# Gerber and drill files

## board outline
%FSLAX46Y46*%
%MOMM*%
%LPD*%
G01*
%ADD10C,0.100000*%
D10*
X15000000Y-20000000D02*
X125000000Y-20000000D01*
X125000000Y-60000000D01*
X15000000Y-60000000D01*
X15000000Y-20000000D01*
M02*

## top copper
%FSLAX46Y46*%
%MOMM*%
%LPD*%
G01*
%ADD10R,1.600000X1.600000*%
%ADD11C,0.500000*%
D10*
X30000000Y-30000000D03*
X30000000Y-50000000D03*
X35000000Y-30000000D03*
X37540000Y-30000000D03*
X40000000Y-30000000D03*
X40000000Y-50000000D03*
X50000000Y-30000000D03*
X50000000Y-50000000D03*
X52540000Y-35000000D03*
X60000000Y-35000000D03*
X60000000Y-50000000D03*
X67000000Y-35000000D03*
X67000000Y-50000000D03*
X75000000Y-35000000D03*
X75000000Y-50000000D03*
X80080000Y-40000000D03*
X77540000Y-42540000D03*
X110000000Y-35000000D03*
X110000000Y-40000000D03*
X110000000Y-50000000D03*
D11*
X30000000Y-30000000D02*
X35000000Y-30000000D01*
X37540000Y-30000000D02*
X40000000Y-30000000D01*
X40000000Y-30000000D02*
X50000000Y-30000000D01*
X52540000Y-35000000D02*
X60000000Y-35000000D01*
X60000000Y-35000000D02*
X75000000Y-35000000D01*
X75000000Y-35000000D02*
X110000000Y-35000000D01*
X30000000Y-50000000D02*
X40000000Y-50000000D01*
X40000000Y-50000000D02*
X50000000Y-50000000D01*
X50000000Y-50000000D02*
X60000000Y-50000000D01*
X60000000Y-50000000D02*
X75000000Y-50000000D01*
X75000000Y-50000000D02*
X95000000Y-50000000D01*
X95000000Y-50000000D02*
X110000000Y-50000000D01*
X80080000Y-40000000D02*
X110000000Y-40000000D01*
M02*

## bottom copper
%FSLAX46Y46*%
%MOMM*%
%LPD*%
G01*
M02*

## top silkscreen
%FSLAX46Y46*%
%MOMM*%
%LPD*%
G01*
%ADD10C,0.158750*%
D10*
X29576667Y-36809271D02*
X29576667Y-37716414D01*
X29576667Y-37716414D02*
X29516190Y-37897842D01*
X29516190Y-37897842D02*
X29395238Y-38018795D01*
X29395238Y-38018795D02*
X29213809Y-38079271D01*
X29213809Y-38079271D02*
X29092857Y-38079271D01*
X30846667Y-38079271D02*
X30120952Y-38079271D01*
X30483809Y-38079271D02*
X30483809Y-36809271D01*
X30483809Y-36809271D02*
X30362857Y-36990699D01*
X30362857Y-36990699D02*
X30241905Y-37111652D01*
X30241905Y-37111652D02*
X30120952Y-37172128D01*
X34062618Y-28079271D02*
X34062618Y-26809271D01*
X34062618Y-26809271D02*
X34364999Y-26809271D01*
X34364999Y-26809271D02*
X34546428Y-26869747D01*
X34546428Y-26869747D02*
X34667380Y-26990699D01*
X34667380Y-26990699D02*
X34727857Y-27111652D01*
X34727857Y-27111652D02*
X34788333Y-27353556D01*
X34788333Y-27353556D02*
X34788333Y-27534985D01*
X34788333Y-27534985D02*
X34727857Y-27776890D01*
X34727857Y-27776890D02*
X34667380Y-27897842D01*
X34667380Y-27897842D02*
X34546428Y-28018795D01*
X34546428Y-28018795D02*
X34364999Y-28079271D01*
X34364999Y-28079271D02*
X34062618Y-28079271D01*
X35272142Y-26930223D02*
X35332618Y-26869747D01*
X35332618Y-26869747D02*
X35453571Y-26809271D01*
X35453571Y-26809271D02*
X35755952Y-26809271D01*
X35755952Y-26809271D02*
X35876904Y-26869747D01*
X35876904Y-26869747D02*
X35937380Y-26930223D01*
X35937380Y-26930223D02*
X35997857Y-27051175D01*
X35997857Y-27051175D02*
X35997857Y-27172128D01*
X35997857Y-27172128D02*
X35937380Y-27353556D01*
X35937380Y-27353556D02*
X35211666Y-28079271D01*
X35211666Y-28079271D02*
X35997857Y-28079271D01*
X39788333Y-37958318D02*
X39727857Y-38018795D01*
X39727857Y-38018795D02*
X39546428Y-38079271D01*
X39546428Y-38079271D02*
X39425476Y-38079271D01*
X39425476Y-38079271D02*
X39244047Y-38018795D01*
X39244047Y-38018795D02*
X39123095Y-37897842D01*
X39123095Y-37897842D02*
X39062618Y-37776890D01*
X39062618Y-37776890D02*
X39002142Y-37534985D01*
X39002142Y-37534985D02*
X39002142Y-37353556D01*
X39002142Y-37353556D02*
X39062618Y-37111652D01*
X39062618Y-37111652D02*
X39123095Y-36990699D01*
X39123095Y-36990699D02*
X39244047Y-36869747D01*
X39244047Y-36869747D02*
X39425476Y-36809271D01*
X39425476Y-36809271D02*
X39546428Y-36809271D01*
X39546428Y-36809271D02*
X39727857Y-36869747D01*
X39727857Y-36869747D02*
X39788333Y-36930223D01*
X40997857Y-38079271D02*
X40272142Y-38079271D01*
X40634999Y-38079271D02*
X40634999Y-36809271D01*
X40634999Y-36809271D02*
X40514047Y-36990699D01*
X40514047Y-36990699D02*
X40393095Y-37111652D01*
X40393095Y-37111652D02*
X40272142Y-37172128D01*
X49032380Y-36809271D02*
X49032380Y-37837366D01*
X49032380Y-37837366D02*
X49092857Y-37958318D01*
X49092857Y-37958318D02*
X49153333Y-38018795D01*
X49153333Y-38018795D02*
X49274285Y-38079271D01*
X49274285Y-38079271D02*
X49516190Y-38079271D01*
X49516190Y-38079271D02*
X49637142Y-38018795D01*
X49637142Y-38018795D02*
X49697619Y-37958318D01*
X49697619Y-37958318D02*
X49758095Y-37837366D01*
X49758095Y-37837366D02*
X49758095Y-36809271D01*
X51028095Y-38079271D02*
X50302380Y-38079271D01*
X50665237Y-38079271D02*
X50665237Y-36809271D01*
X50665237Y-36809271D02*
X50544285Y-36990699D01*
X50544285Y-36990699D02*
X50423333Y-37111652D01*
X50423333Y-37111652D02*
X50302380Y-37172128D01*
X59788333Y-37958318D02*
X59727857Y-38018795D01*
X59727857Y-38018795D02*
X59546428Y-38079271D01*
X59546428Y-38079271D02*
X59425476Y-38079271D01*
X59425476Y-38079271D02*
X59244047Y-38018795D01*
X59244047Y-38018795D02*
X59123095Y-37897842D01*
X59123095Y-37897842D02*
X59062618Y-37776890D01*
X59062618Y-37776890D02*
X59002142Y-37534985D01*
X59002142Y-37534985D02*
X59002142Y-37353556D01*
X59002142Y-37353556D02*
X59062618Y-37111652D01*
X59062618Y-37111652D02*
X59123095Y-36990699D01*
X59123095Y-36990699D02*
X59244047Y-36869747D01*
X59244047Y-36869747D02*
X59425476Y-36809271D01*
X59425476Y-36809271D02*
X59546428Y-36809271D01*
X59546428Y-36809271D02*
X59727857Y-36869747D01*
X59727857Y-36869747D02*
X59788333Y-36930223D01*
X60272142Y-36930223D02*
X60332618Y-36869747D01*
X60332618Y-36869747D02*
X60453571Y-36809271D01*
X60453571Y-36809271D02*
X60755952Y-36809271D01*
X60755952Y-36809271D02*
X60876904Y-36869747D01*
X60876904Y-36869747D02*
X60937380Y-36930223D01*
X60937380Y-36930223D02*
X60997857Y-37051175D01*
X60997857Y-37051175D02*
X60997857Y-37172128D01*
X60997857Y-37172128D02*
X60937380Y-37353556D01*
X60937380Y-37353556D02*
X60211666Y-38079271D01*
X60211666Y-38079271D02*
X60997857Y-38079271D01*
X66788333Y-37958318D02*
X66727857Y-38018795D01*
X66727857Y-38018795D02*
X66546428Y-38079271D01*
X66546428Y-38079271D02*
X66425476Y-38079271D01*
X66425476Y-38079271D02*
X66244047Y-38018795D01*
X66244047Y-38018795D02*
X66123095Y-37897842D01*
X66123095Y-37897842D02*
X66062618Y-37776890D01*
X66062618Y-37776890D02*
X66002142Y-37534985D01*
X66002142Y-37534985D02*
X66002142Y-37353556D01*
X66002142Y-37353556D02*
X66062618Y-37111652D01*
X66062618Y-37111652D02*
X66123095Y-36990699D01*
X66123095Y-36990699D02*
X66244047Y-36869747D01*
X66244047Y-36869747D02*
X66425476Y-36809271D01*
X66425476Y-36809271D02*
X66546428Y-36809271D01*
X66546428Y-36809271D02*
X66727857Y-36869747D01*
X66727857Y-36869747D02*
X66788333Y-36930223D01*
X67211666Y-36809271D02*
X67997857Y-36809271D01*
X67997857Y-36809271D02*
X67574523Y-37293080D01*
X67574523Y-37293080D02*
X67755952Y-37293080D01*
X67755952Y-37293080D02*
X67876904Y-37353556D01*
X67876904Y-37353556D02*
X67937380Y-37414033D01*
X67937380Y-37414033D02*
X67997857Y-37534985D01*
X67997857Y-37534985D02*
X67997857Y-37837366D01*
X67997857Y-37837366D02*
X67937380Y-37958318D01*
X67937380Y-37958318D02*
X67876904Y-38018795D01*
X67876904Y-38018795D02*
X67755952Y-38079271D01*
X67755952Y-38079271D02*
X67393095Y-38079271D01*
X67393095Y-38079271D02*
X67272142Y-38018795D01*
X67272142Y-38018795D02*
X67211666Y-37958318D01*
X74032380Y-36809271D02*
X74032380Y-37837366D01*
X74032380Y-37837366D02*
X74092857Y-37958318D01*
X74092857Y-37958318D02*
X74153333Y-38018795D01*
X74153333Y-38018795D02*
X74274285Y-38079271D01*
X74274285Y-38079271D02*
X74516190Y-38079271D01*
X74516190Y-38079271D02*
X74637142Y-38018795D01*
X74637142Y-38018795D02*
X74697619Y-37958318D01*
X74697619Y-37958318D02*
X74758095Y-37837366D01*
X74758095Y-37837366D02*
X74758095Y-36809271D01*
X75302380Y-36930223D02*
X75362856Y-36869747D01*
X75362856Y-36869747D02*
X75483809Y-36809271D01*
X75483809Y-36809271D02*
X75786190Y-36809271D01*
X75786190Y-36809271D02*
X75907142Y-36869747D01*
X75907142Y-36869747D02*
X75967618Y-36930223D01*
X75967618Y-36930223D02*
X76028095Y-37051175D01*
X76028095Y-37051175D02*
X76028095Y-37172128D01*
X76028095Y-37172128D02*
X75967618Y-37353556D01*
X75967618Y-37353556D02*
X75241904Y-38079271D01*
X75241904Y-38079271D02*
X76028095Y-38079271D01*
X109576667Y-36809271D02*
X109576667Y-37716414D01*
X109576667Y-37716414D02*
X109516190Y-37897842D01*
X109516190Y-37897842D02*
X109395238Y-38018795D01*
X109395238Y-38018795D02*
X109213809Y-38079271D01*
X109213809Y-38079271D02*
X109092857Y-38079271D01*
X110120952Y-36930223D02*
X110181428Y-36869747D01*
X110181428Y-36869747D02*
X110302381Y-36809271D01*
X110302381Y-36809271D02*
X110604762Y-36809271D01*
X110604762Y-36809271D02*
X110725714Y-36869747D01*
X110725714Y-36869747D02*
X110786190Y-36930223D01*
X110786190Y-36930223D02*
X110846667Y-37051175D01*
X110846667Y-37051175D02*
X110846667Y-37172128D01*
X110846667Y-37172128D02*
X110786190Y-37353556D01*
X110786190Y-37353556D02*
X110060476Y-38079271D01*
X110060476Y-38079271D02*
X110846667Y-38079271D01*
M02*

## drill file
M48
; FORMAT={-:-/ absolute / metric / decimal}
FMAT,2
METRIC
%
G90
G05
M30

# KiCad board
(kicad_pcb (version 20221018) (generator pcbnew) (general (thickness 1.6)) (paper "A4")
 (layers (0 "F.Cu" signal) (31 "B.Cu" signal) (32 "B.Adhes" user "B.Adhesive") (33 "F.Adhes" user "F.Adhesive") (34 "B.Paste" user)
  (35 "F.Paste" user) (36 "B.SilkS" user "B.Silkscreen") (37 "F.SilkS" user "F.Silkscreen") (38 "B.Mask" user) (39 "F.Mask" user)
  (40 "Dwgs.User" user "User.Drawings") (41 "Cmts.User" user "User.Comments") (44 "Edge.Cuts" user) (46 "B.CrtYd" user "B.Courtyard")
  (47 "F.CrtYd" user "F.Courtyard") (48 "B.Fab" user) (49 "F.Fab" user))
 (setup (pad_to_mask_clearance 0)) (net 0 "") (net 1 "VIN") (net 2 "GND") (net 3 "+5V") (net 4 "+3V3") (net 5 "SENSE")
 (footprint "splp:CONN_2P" (layer "F.Cu") (at 30 40)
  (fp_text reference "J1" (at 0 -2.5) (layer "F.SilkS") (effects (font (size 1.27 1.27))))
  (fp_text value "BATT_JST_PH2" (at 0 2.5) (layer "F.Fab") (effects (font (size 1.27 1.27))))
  (pad "1" smd rect (at 0 -10) (size 1.6 1.6) (layers "F.Cu" "F.Paste" "F.Mask") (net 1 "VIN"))
  (pad "2" smd rect (at 0 10) (size 1.6 1.6) (layers "F.Cu" "F.Paste" "F.Mask") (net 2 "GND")))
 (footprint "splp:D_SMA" (layer "F.Cu") (at 35 30)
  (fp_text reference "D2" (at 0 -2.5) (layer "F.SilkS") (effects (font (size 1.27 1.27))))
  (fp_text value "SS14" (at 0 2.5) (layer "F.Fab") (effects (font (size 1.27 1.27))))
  (pad "1" smd rect (at 0 0) (size 1.6 1.6) (layers "F.Cu" "F.Paste" "F.Mask") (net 1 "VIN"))
  (pad "2" smd rect (at 2.54 0) (size 1.6 1.6) (layers "F.Cu" "F.Paste" "F.Mask") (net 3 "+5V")))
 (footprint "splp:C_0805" (layer "F.Cu") (at 40 40)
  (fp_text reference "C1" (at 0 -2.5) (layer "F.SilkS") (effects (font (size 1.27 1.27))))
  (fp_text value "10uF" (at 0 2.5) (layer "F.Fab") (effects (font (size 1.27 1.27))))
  (pad "1" smd rect (at 0 -10) (size 1.6 1.6) (layers "F.Cu" "F.Paste" "F.Mask") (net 3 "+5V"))
  (pad "2" smd rect (at 0 10) (size 1.6 1.6) (layers "F.Cu" "F.Paste" "F.Mask") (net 2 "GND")))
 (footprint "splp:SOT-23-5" (layer "F.Cu") (at 50 40)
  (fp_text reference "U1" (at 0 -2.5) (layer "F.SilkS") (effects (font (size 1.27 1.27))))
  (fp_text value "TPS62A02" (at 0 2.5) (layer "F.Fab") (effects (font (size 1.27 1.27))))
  (pad "1" smd rect (at 0 -10) (size 1.6 1.6) (layers "F.Cu" "F.Paste" "F.Mask") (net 3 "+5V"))
  (pad "2" smd rect (at 0 10) (size 1.6 1.6) (layers "F.Cu" "F.Paste" "F.Mask") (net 2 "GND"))
  (pad "3" smd rect (at 2.54 -5) (size 1.6 1.6) (layers "F.Cu" "F.Paste" "F.Mask") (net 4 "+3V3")))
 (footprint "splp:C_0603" (layer "F.Cu") (at 60 40)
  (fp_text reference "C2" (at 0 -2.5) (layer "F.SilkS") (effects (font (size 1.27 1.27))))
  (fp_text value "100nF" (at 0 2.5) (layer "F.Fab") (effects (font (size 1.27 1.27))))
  (pad "1" smd rect (at 0 -5) (size 1.6 1.6) (layers "F.Cu" "F.Paste" "F.Mask") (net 4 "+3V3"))
  (pad "2" smd rect (at 0 10) (size 1.6 1.6) (layers "F.Cu" "F.Paste" "F.Mask") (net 2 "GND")))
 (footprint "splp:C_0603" (layer "F.Cu") (at 67 40)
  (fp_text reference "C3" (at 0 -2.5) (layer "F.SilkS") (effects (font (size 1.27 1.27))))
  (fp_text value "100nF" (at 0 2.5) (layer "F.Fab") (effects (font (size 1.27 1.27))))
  (pad "1" smd rect (at 0 -5) (size 1.6 1.6) (layers "F.Cu" "F.Paste" "F.Mask") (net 4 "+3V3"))
  (pad "2" smd rect (at 0 10) (size 1.6 1.6) (layers "F.Cu" "F.Paste" "F.Mask") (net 2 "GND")))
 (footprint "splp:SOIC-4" (layer "F.Cu") (at 75 40)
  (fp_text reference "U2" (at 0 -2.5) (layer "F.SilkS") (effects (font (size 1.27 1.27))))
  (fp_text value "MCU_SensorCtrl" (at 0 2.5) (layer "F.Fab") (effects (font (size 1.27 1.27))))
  (pad "1" smd rect (at 0 -5) (size 1.6 1.6) (layers "F.Cu" "F.Paste" "F.Mask") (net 4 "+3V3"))
  (pad "2" smd rect (at 0 10) (size 1.6 1.6) (layers "F.Cu" "F.Paste" "F.Mask") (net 2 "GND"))
  (pad "3" smd rect (at 5.08 0) (size 1.6 1.6) (layers "F.Cu" "F.Paste" "F.Mask") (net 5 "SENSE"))
  (pad "4" smd rect (at 2.54 2.54) (size 1.6 1.6) (layers "F.Cu" "F.Paste" "F.Mask")))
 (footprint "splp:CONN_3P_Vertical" (layer "F.Cu") (at 110 40)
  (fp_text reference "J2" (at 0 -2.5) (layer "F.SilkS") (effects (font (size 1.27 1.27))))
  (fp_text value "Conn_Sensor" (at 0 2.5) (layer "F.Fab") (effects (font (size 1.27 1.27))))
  (pad "1" smd rect (at 0 -5) (size 1.6 1.6) (layers "F.Cu" "F.Paste" "F.Mask") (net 4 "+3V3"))
  (pad "2" smd rect (at 0 0) (size 1.6 1.6) (layers "F.Cu" "F.Paste" "F.Mask") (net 5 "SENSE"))
  (pad "3" smd rect (at 0 10) (size 1.6 1.6) (layers "F.Cu" "F.Paste" "F.Mask") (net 2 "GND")))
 (segment (start 30 30) (end 35 30) (width 0.5) (layer "F.Cu") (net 1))
 (segment (start 37.54 30) (end 40 30) (width 0.5) (layer "F.Cu") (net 3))
 (segment (start 40 30) (end 50 30) (width 0.5) (layer "F.Cu") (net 3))
 (segment (start 52.54 35) (end 60 35) (width 0.5) (layer "F.Cu") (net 4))
 (segment (start 60 35) (end 75 35) (width 0.5) (layer "F.Cu") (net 4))
 (segment (start 75 35) (end 110 35) (width 0.5) (layer "F.Cu") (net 4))
 (segment (start 30 50) (end 40 50) (width 0.5) (layer "F.Cu") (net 2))
 (segment (start 40 50) (end 50 50) (width 0.5) (layer "F.Cu") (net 2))
 (segment (start 50 50) (end 60 50) (width 0.5) (layer "F.Cu") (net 2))
 (segment (start 60 50) (end 75 50) (width 0.5) (layer "F.Cu") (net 2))
 (segment (start 75 50) (end 95 50) (width 0.5) (layer "F.Cu") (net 2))
 (segment (start 95 50) (end 110 50) (width 0.5) (layer "F.Cu") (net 2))
 (segment (start 80.08 40) (end 110 40) (width 0.5) (layer "F.Cu") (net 5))
 (gr_rect (start 15 20) (end 125 60) (stroke (width 0.1) (type default)) (fill none) (layer "Edge.Cuts")))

